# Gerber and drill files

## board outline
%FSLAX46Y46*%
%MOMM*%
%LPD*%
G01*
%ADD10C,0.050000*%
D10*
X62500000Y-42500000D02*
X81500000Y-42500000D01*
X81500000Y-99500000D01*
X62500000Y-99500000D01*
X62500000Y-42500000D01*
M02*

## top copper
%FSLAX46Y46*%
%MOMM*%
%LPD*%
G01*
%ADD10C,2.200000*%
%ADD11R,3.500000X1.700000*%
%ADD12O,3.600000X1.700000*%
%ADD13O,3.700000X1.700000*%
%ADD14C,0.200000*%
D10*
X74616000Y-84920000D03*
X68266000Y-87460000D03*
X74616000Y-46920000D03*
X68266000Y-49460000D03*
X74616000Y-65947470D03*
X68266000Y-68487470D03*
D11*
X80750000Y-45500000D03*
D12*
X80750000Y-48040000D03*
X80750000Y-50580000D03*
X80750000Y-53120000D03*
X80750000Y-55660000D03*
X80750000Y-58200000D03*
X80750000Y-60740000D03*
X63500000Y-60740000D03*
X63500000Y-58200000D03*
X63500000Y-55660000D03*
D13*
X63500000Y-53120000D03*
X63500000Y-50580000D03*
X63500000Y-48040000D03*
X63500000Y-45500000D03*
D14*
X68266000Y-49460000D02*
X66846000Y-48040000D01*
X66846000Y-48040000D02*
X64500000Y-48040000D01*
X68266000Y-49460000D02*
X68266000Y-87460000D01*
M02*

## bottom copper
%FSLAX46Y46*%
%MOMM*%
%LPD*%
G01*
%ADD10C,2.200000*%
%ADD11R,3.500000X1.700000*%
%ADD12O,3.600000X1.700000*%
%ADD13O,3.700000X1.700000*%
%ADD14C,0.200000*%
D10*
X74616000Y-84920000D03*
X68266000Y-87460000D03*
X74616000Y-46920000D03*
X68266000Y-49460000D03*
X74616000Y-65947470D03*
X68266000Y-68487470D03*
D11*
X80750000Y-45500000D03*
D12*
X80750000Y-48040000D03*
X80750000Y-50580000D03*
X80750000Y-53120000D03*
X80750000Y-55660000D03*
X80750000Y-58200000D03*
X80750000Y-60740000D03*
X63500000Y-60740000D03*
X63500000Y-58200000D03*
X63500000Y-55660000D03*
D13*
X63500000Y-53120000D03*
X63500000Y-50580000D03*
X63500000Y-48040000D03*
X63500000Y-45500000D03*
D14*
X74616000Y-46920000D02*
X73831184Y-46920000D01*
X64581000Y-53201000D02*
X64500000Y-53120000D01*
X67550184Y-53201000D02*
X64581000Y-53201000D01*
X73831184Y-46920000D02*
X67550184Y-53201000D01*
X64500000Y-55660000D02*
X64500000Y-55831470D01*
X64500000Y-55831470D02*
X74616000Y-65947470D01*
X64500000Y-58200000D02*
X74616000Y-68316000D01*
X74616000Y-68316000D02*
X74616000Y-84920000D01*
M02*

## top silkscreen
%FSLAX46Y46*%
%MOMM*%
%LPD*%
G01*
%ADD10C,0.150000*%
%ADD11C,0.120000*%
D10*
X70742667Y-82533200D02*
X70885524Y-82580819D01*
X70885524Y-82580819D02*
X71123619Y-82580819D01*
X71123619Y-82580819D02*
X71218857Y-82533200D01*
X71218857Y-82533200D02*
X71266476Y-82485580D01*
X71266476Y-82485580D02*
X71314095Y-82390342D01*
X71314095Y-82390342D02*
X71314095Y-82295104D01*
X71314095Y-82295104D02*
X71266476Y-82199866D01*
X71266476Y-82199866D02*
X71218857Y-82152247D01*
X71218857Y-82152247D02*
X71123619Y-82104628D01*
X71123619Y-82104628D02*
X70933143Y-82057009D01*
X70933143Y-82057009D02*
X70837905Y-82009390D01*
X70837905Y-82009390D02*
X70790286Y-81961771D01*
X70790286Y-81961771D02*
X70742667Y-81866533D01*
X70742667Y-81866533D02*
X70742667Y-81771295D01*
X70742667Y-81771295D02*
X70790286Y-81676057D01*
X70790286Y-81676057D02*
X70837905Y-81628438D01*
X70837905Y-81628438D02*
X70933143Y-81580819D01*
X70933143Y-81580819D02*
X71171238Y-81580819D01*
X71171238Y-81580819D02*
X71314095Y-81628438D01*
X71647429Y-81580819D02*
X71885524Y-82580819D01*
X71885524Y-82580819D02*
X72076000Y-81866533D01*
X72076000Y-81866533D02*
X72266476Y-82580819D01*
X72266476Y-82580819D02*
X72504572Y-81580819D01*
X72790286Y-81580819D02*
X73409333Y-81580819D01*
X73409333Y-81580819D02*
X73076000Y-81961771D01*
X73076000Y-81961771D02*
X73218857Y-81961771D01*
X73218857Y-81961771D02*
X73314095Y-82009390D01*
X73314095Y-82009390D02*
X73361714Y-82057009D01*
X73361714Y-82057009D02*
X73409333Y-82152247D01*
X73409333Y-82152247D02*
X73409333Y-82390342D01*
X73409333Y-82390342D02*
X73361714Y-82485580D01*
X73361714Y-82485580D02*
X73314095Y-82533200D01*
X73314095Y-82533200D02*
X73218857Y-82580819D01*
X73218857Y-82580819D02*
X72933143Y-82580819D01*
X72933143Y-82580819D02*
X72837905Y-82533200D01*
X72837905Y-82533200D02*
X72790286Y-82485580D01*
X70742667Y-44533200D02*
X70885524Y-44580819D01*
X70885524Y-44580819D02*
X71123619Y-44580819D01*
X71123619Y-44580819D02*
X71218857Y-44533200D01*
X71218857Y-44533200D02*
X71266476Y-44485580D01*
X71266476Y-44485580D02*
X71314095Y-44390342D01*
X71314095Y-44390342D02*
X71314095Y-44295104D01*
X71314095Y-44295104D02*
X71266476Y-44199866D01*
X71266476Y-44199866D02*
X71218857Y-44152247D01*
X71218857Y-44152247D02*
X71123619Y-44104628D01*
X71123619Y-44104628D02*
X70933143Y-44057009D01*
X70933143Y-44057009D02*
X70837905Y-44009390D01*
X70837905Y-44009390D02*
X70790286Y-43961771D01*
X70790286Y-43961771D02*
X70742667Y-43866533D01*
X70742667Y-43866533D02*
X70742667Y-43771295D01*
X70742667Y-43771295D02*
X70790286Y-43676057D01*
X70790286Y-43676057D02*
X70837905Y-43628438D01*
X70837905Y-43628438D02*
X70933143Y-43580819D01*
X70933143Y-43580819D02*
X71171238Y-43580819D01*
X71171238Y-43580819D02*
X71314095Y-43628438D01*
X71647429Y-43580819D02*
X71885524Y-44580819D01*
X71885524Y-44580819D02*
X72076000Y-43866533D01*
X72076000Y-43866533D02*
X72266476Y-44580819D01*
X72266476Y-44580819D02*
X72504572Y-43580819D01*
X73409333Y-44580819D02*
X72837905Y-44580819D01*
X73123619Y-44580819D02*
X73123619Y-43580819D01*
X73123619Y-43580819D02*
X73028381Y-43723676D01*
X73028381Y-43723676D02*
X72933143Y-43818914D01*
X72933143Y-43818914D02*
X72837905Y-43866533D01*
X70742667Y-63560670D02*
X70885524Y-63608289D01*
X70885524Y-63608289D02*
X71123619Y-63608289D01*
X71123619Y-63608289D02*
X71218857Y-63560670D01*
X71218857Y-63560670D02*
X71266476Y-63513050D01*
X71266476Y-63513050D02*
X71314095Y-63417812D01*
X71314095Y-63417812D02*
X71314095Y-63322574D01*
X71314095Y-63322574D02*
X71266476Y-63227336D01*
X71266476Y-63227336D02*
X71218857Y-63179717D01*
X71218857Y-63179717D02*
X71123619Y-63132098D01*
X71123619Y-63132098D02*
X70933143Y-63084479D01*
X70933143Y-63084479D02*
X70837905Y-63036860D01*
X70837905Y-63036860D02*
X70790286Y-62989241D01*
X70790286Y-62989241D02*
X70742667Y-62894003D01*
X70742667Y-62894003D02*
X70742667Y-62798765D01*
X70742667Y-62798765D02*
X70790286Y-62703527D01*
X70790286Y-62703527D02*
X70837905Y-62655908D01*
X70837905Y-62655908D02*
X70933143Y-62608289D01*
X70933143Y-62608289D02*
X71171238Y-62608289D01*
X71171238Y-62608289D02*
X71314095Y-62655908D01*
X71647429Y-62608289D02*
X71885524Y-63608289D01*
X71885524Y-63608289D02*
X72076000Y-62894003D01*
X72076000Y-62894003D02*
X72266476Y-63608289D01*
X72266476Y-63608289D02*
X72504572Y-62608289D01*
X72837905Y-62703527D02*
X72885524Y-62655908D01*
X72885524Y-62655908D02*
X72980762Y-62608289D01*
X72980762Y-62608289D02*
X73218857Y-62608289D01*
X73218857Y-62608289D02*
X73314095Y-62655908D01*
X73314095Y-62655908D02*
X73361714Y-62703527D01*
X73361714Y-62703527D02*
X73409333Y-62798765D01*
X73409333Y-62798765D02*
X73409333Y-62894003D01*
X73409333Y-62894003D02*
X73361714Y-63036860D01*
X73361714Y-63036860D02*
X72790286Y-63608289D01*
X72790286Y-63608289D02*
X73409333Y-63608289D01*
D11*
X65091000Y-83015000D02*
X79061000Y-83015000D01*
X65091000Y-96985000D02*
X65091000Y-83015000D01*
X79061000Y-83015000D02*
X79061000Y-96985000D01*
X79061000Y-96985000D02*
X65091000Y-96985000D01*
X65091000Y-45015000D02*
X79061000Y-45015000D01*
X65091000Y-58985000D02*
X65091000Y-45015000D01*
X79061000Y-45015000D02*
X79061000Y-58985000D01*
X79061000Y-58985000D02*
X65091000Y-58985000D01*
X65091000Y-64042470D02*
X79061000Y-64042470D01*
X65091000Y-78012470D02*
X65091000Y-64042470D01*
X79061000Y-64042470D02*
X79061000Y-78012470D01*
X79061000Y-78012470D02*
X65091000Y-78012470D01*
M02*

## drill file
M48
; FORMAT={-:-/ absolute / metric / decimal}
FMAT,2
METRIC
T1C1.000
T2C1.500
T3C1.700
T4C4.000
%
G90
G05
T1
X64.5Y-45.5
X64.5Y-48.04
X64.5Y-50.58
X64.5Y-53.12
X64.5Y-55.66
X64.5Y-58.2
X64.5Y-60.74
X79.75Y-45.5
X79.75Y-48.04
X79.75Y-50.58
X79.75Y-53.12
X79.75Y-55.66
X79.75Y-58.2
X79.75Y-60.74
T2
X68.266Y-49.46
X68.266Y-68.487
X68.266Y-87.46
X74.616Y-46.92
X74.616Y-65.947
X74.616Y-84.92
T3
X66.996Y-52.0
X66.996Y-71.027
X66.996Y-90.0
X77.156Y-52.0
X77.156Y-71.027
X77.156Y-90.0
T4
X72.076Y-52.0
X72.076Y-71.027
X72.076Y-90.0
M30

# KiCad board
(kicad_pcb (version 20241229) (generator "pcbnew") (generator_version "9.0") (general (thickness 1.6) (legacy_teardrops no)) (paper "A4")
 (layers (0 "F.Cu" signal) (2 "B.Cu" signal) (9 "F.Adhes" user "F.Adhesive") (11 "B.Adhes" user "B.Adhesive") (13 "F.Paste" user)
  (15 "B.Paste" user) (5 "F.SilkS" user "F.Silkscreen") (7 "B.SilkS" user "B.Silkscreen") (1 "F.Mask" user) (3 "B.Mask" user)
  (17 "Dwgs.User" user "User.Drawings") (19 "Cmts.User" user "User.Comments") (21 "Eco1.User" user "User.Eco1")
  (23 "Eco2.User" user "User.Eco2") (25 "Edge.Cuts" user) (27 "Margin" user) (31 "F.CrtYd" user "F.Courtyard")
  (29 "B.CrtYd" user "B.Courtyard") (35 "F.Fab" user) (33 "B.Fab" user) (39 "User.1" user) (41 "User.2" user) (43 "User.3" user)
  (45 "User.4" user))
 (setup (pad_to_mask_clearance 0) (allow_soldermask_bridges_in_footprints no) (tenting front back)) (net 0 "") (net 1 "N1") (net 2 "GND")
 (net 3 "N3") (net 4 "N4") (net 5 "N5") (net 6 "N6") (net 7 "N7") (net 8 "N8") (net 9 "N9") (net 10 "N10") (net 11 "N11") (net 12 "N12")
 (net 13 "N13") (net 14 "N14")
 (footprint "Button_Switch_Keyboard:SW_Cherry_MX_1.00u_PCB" (layer "F.Cu") (at 74.616 84.92)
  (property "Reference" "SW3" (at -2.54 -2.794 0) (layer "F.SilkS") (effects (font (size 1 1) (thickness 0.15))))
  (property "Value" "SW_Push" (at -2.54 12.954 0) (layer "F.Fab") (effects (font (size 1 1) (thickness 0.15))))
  (fp_line (start -9.525 -1.905) (end 4.445 -1.905) (stroke (width 0.12) (type solid)) (layer "F.SilkS"))
  (fp_line (start -9.525 12.065) (end -9.525 -1.905) (stroke (width 0.12) (type solid)) (layer "F.SilkS"))
  (fp_line (start 4.445 -1.905) (end 4.445 12.065) (stroke (width 0.12) (type solid)) (layer "F.SilkS"))
  (fp_line (start 4.445 12.065) (end -9.525 12.065) (stroke (width 0.12) (type solid)) (layer "F.SilkS"))
  (pad "" np_thru_hole circle (at -7.62 5.08) (size 1.7 1.7) (drill 1.7) (layers "*.Cu" "*.Mask"))
  (pad "" np_thru_hole circle (at -2.54 5.08) (size 4 4) (drill 4) (layers "*.Cu" "*.Mask"))
  (pad "" np_thru_hole circle (at 2.54 5.08) (size 1.7 1.7) (drill 1.7) (layers "*.Cu" "*.Mask"))
  (pad "1" thru_hole circle (at 0 0) (size 2.2 2.2) (drill 1.5) (layers "*.Cu" "*.Mask") (remove_unused_layers no) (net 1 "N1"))
  (pad "2" thru_hole circle (at -6.35 2.54) (size 2.2 2.2) (drill 1.5) (layers "*.Cu" "*.Mask") (remove_unused_layers no) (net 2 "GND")))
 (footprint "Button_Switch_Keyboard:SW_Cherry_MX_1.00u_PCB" (layer "F.Cu") (at 74.616 46.92)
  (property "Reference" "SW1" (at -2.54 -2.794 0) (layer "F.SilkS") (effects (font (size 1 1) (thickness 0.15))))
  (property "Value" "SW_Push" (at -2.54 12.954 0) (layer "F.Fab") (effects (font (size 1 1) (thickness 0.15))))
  (fp_line (start -9.525 -1.905) (end 4.445 -1.905) (stroke (width 0.12) (type solid)) (layer "F.SilkS"))
  (fp_line (start -9.525 12.065) (end -9.525 -1.905) (stroke (width 0.12) (type solid)) (layer "F.SilkS"))
  (fp_line (start 4.445 -1.905) (end 4.445 12.065) (stroke (width 0.12) (type solid)) (layer "F.SilkS"))
  (fp_line (start 4.445 12.065) (end -9.525 12.065) (stroke (width 0.12) (type solid)) (layer "F.SilkS"))
  (pad "" np_thru_hole circle (at -7.62 5.08) (size 1.7 1.7) (drill 1.7) (layers "*.Cu" "*.Mask"))
  (pad "" np_thru_hole circle (at -2.54 5.08) (size 4 4) (drill 4) (layers "*.Cu" "*.Mask"))
  (pad "" np_thru_hole circle (at 2.54 5.08) (size 1.7 1.7) (drill 1.7) (layers "*.Cu" "*.Mask"))
  (pad "1" thru_hole circle (at 0 0) (size 2.2 2.2) (drill 1.5) (layers "*.Cu" "*.Mask") (remove_unused_layers no) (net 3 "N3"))
  (pad "2" thru_hole circle (at -6.35 2.54) (size 2.2 2.2) (drill 1.5) (layers "*.Cu" "*.Mask") (remove_unused_layers no) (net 2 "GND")))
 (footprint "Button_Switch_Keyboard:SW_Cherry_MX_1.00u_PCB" (layer "F.Cu") (at 74.616 65.94747)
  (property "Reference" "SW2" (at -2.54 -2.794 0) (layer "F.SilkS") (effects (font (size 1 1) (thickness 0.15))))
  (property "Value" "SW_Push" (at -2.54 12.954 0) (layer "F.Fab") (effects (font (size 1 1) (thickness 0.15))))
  (fp_line (start -9.525 -1.905) (end 4.445 -1.905) (stroke (width 0.12) (type solid)) (layer "F.SilkS"))
  (fp_line (start -9.525 12.065) (end -9.525 -1.905) (stroke (width 0.12) (type solid)) (layer "F.SilkS"))
  (fp_line (start 4.445 -1.905) (end 4.445 12.065) (stroke (width 0.12) (type solid)) (layer "F.SilkS"))
  (fp_line (start 4.445 12.065) (end -9.525 12.065) (stroke (width 0.12) (type solid)) (layer "F.SilkS"))
  (pad "" np_thru_hole circle (at -7.62 5.08) (size 1.7 1.7) (drill 1.7) (layers "*.Cu" "*.Mask"))
  (pad "" np_thru_hole circle (at -2.54 5.08) (size 4 4) (drill 4) (layers "*.Cu" "*.Mask"))
  (pad "" np_thru_hole circle (at 2.54 5.08) (size 1.7 1.7) (drill 1.7) (layers "*.Cu" "*.Mask"))
  (pad "1" thru_hole circle (at 0 0) (size 2.2 2.2) (drill 1.5) (layers "*.Cu" "*.Mask") (remove_unused_layers no) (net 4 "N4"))
  (pad "2" thru_hole circle (at -6.35 2.54) (size 2.2 2.2) (drill 1.5) (layers "*.Cu" "*.Mask") (remove_unused_layers no) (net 2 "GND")))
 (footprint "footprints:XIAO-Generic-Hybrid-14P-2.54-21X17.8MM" (layer "B.Cu") (at 72.125 53.12 180)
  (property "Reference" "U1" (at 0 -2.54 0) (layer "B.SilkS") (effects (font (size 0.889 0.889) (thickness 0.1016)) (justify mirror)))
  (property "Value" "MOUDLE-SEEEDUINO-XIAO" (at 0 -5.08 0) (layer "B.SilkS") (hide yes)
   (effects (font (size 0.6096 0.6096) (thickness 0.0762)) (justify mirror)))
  (pad "1" thru_hole rect (at -7.625 7.62 180) (size 3.5 1.7) (drill 1 (offset -1 0)) (layers "*.Cu" "*.Mask") (remove_unused_layers no)
   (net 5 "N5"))
  (pad "2" thru_hole oval (at -7.625 5.08 180) (size 3.6 1.7) (drill 1 (offset -1 0)) (layers "*.Cu" "*.Mask") (remove_unused_layers no)
   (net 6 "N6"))
  (pad "3" thru_hole oval (at -7.625 2.54 180) (size 3.6 1.7) (drill 1 (offset -1 0)) (layers "*.Cu" "*.Mask") (remove_unused_layers no)
   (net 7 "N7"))
  (pad "4" thru_hole oval (at -7.625 0 180) (size 3.6 1.7) (drill 1 (offset -1 0)) (layers "*.Cu" "*.Mask") (remove_unused_layers no)
   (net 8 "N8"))
  (pad "5" thru_hole oval (at -7.625 -2.54 180) (size 3.6 1.7) (drill 1 (offset -1 0)) (layers "*.Cu" "*.Mask") (remove_unused_layers no)
   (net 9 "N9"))
  (pad "6" thru_hole oval (at -7.625 -5.08) (size 3.6 1.7) (drill 1 (offset 1 0)) (layers "*.Cu" "*.Mask") (remove_unused_layers no)
   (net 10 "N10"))
  (pad "7" thru_hole oval (at -7.625 -7.62 180) (size 3.6 1.7) (drill 1 (offset -1 0)) (layers "*.Cu" "*.Mask") (remove_unused_layers no)
   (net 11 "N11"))
  (pad "8" thru_hole oval (at 7.625 -7.62 180) (size 3.6 1.7) (drill 1 (offset 1 0)) (layers "*.Cu" "*.Mask") (remove_unused_layers no)
   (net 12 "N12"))
  (pad "9" thru_hole oval (at 7.625 -5.08 180) (size 3.6 1.7) (drill 1 (offset 1 0)) (layers "*.Cu" "*.Mask") (remove_unused_layers no)
   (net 1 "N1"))
  (pad "10" thru_hole oval (at 7.625 -2.54 180) (size 3.6 1.7) (drill 1 (offset 1 0)) (layers "*.Cu" "*.Mask") (remove_unused_layers no)
   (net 4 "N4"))
  (pad "11" thru_hole oval (at 7.625 0 180) (size 3.7 1.7) (drill 1 (offset 1 0)) (layers "*.Cu" "*.Mask") (remove_unused_layers no)
   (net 3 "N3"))
  (pad "12" thru_hole oval (at 7.625 2.54 180) (size 3.7 1.7) (drill 1 (offset 1 0)) (layers "*.Cu" "*.Mask") (remove_unused_layers no)
   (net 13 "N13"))
  (pad "13" thru_hole oval (at 7.625 5.08 180) (size 3.7 1.7) (drill 1 (offset 1 0)) (layers "*.Cu" "*.Mask") (remove_unused_layers no)
   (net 2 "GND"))
  (pad "14" thru_hole oval (at 7.625 7.62 180) (size 3.7 1.7) (drill 1 (offset 1 0)) (layers "*.Cu" "*.Mask") (remove_unused_layers no)
   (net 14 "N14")))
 (gr_rect (start 62.5 42.5) (end 81.5 99.5) (stroke (width 0.05) (type default)) (fill no) (layer "Edge.Cuts"))
 (segment (start 68.266 49.46) (end 66.846 48.04) (width 0.2) (layer "F.Cu") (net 2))
 (segment (start 66.846 48.04) (end 64.5 48.04) (width 0.2) (layer "F.Cu") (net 2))
 (segment (start 68.266 49.46) (end 68.266 87.46) (width 0.2) (layer "F.Cu") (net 2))
 (segment (start 74.616 46.92) (end 73.831184 46.92) (width 0.2) (layer "B.Cu") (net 3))
 (segment (start 64.581 53.201) (end 64.5 53.12) (width 0.2) (layer "B.Cu") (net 3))
 (segment (start 67.550184 53.201) (end 64.581 53.201) (width 0.2) (layer "B.Cu") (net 3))
 (segment (start 73.831184 46.92) (end 67.550184 53.201) (width 0.2) (layer "B.Cu") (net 3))
 (segment (start 64.5 55.66) (end 64.5 55.83147) (width 0.2) (layer "B.Cu") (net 4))
 (segment (start 64.5 55.83147) (end 74.616 65.94747) (width 0.2) (layer "B.Cu") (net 4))
 (segment (start 64.5 58.2) (end 74.616 68.316) (width 0.2) (layer "B.Cu") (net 1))
 (segment (start 74.616 68.316) (end 74.616 84.92) (width 0.2) (layer "B.Cu") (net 1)))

